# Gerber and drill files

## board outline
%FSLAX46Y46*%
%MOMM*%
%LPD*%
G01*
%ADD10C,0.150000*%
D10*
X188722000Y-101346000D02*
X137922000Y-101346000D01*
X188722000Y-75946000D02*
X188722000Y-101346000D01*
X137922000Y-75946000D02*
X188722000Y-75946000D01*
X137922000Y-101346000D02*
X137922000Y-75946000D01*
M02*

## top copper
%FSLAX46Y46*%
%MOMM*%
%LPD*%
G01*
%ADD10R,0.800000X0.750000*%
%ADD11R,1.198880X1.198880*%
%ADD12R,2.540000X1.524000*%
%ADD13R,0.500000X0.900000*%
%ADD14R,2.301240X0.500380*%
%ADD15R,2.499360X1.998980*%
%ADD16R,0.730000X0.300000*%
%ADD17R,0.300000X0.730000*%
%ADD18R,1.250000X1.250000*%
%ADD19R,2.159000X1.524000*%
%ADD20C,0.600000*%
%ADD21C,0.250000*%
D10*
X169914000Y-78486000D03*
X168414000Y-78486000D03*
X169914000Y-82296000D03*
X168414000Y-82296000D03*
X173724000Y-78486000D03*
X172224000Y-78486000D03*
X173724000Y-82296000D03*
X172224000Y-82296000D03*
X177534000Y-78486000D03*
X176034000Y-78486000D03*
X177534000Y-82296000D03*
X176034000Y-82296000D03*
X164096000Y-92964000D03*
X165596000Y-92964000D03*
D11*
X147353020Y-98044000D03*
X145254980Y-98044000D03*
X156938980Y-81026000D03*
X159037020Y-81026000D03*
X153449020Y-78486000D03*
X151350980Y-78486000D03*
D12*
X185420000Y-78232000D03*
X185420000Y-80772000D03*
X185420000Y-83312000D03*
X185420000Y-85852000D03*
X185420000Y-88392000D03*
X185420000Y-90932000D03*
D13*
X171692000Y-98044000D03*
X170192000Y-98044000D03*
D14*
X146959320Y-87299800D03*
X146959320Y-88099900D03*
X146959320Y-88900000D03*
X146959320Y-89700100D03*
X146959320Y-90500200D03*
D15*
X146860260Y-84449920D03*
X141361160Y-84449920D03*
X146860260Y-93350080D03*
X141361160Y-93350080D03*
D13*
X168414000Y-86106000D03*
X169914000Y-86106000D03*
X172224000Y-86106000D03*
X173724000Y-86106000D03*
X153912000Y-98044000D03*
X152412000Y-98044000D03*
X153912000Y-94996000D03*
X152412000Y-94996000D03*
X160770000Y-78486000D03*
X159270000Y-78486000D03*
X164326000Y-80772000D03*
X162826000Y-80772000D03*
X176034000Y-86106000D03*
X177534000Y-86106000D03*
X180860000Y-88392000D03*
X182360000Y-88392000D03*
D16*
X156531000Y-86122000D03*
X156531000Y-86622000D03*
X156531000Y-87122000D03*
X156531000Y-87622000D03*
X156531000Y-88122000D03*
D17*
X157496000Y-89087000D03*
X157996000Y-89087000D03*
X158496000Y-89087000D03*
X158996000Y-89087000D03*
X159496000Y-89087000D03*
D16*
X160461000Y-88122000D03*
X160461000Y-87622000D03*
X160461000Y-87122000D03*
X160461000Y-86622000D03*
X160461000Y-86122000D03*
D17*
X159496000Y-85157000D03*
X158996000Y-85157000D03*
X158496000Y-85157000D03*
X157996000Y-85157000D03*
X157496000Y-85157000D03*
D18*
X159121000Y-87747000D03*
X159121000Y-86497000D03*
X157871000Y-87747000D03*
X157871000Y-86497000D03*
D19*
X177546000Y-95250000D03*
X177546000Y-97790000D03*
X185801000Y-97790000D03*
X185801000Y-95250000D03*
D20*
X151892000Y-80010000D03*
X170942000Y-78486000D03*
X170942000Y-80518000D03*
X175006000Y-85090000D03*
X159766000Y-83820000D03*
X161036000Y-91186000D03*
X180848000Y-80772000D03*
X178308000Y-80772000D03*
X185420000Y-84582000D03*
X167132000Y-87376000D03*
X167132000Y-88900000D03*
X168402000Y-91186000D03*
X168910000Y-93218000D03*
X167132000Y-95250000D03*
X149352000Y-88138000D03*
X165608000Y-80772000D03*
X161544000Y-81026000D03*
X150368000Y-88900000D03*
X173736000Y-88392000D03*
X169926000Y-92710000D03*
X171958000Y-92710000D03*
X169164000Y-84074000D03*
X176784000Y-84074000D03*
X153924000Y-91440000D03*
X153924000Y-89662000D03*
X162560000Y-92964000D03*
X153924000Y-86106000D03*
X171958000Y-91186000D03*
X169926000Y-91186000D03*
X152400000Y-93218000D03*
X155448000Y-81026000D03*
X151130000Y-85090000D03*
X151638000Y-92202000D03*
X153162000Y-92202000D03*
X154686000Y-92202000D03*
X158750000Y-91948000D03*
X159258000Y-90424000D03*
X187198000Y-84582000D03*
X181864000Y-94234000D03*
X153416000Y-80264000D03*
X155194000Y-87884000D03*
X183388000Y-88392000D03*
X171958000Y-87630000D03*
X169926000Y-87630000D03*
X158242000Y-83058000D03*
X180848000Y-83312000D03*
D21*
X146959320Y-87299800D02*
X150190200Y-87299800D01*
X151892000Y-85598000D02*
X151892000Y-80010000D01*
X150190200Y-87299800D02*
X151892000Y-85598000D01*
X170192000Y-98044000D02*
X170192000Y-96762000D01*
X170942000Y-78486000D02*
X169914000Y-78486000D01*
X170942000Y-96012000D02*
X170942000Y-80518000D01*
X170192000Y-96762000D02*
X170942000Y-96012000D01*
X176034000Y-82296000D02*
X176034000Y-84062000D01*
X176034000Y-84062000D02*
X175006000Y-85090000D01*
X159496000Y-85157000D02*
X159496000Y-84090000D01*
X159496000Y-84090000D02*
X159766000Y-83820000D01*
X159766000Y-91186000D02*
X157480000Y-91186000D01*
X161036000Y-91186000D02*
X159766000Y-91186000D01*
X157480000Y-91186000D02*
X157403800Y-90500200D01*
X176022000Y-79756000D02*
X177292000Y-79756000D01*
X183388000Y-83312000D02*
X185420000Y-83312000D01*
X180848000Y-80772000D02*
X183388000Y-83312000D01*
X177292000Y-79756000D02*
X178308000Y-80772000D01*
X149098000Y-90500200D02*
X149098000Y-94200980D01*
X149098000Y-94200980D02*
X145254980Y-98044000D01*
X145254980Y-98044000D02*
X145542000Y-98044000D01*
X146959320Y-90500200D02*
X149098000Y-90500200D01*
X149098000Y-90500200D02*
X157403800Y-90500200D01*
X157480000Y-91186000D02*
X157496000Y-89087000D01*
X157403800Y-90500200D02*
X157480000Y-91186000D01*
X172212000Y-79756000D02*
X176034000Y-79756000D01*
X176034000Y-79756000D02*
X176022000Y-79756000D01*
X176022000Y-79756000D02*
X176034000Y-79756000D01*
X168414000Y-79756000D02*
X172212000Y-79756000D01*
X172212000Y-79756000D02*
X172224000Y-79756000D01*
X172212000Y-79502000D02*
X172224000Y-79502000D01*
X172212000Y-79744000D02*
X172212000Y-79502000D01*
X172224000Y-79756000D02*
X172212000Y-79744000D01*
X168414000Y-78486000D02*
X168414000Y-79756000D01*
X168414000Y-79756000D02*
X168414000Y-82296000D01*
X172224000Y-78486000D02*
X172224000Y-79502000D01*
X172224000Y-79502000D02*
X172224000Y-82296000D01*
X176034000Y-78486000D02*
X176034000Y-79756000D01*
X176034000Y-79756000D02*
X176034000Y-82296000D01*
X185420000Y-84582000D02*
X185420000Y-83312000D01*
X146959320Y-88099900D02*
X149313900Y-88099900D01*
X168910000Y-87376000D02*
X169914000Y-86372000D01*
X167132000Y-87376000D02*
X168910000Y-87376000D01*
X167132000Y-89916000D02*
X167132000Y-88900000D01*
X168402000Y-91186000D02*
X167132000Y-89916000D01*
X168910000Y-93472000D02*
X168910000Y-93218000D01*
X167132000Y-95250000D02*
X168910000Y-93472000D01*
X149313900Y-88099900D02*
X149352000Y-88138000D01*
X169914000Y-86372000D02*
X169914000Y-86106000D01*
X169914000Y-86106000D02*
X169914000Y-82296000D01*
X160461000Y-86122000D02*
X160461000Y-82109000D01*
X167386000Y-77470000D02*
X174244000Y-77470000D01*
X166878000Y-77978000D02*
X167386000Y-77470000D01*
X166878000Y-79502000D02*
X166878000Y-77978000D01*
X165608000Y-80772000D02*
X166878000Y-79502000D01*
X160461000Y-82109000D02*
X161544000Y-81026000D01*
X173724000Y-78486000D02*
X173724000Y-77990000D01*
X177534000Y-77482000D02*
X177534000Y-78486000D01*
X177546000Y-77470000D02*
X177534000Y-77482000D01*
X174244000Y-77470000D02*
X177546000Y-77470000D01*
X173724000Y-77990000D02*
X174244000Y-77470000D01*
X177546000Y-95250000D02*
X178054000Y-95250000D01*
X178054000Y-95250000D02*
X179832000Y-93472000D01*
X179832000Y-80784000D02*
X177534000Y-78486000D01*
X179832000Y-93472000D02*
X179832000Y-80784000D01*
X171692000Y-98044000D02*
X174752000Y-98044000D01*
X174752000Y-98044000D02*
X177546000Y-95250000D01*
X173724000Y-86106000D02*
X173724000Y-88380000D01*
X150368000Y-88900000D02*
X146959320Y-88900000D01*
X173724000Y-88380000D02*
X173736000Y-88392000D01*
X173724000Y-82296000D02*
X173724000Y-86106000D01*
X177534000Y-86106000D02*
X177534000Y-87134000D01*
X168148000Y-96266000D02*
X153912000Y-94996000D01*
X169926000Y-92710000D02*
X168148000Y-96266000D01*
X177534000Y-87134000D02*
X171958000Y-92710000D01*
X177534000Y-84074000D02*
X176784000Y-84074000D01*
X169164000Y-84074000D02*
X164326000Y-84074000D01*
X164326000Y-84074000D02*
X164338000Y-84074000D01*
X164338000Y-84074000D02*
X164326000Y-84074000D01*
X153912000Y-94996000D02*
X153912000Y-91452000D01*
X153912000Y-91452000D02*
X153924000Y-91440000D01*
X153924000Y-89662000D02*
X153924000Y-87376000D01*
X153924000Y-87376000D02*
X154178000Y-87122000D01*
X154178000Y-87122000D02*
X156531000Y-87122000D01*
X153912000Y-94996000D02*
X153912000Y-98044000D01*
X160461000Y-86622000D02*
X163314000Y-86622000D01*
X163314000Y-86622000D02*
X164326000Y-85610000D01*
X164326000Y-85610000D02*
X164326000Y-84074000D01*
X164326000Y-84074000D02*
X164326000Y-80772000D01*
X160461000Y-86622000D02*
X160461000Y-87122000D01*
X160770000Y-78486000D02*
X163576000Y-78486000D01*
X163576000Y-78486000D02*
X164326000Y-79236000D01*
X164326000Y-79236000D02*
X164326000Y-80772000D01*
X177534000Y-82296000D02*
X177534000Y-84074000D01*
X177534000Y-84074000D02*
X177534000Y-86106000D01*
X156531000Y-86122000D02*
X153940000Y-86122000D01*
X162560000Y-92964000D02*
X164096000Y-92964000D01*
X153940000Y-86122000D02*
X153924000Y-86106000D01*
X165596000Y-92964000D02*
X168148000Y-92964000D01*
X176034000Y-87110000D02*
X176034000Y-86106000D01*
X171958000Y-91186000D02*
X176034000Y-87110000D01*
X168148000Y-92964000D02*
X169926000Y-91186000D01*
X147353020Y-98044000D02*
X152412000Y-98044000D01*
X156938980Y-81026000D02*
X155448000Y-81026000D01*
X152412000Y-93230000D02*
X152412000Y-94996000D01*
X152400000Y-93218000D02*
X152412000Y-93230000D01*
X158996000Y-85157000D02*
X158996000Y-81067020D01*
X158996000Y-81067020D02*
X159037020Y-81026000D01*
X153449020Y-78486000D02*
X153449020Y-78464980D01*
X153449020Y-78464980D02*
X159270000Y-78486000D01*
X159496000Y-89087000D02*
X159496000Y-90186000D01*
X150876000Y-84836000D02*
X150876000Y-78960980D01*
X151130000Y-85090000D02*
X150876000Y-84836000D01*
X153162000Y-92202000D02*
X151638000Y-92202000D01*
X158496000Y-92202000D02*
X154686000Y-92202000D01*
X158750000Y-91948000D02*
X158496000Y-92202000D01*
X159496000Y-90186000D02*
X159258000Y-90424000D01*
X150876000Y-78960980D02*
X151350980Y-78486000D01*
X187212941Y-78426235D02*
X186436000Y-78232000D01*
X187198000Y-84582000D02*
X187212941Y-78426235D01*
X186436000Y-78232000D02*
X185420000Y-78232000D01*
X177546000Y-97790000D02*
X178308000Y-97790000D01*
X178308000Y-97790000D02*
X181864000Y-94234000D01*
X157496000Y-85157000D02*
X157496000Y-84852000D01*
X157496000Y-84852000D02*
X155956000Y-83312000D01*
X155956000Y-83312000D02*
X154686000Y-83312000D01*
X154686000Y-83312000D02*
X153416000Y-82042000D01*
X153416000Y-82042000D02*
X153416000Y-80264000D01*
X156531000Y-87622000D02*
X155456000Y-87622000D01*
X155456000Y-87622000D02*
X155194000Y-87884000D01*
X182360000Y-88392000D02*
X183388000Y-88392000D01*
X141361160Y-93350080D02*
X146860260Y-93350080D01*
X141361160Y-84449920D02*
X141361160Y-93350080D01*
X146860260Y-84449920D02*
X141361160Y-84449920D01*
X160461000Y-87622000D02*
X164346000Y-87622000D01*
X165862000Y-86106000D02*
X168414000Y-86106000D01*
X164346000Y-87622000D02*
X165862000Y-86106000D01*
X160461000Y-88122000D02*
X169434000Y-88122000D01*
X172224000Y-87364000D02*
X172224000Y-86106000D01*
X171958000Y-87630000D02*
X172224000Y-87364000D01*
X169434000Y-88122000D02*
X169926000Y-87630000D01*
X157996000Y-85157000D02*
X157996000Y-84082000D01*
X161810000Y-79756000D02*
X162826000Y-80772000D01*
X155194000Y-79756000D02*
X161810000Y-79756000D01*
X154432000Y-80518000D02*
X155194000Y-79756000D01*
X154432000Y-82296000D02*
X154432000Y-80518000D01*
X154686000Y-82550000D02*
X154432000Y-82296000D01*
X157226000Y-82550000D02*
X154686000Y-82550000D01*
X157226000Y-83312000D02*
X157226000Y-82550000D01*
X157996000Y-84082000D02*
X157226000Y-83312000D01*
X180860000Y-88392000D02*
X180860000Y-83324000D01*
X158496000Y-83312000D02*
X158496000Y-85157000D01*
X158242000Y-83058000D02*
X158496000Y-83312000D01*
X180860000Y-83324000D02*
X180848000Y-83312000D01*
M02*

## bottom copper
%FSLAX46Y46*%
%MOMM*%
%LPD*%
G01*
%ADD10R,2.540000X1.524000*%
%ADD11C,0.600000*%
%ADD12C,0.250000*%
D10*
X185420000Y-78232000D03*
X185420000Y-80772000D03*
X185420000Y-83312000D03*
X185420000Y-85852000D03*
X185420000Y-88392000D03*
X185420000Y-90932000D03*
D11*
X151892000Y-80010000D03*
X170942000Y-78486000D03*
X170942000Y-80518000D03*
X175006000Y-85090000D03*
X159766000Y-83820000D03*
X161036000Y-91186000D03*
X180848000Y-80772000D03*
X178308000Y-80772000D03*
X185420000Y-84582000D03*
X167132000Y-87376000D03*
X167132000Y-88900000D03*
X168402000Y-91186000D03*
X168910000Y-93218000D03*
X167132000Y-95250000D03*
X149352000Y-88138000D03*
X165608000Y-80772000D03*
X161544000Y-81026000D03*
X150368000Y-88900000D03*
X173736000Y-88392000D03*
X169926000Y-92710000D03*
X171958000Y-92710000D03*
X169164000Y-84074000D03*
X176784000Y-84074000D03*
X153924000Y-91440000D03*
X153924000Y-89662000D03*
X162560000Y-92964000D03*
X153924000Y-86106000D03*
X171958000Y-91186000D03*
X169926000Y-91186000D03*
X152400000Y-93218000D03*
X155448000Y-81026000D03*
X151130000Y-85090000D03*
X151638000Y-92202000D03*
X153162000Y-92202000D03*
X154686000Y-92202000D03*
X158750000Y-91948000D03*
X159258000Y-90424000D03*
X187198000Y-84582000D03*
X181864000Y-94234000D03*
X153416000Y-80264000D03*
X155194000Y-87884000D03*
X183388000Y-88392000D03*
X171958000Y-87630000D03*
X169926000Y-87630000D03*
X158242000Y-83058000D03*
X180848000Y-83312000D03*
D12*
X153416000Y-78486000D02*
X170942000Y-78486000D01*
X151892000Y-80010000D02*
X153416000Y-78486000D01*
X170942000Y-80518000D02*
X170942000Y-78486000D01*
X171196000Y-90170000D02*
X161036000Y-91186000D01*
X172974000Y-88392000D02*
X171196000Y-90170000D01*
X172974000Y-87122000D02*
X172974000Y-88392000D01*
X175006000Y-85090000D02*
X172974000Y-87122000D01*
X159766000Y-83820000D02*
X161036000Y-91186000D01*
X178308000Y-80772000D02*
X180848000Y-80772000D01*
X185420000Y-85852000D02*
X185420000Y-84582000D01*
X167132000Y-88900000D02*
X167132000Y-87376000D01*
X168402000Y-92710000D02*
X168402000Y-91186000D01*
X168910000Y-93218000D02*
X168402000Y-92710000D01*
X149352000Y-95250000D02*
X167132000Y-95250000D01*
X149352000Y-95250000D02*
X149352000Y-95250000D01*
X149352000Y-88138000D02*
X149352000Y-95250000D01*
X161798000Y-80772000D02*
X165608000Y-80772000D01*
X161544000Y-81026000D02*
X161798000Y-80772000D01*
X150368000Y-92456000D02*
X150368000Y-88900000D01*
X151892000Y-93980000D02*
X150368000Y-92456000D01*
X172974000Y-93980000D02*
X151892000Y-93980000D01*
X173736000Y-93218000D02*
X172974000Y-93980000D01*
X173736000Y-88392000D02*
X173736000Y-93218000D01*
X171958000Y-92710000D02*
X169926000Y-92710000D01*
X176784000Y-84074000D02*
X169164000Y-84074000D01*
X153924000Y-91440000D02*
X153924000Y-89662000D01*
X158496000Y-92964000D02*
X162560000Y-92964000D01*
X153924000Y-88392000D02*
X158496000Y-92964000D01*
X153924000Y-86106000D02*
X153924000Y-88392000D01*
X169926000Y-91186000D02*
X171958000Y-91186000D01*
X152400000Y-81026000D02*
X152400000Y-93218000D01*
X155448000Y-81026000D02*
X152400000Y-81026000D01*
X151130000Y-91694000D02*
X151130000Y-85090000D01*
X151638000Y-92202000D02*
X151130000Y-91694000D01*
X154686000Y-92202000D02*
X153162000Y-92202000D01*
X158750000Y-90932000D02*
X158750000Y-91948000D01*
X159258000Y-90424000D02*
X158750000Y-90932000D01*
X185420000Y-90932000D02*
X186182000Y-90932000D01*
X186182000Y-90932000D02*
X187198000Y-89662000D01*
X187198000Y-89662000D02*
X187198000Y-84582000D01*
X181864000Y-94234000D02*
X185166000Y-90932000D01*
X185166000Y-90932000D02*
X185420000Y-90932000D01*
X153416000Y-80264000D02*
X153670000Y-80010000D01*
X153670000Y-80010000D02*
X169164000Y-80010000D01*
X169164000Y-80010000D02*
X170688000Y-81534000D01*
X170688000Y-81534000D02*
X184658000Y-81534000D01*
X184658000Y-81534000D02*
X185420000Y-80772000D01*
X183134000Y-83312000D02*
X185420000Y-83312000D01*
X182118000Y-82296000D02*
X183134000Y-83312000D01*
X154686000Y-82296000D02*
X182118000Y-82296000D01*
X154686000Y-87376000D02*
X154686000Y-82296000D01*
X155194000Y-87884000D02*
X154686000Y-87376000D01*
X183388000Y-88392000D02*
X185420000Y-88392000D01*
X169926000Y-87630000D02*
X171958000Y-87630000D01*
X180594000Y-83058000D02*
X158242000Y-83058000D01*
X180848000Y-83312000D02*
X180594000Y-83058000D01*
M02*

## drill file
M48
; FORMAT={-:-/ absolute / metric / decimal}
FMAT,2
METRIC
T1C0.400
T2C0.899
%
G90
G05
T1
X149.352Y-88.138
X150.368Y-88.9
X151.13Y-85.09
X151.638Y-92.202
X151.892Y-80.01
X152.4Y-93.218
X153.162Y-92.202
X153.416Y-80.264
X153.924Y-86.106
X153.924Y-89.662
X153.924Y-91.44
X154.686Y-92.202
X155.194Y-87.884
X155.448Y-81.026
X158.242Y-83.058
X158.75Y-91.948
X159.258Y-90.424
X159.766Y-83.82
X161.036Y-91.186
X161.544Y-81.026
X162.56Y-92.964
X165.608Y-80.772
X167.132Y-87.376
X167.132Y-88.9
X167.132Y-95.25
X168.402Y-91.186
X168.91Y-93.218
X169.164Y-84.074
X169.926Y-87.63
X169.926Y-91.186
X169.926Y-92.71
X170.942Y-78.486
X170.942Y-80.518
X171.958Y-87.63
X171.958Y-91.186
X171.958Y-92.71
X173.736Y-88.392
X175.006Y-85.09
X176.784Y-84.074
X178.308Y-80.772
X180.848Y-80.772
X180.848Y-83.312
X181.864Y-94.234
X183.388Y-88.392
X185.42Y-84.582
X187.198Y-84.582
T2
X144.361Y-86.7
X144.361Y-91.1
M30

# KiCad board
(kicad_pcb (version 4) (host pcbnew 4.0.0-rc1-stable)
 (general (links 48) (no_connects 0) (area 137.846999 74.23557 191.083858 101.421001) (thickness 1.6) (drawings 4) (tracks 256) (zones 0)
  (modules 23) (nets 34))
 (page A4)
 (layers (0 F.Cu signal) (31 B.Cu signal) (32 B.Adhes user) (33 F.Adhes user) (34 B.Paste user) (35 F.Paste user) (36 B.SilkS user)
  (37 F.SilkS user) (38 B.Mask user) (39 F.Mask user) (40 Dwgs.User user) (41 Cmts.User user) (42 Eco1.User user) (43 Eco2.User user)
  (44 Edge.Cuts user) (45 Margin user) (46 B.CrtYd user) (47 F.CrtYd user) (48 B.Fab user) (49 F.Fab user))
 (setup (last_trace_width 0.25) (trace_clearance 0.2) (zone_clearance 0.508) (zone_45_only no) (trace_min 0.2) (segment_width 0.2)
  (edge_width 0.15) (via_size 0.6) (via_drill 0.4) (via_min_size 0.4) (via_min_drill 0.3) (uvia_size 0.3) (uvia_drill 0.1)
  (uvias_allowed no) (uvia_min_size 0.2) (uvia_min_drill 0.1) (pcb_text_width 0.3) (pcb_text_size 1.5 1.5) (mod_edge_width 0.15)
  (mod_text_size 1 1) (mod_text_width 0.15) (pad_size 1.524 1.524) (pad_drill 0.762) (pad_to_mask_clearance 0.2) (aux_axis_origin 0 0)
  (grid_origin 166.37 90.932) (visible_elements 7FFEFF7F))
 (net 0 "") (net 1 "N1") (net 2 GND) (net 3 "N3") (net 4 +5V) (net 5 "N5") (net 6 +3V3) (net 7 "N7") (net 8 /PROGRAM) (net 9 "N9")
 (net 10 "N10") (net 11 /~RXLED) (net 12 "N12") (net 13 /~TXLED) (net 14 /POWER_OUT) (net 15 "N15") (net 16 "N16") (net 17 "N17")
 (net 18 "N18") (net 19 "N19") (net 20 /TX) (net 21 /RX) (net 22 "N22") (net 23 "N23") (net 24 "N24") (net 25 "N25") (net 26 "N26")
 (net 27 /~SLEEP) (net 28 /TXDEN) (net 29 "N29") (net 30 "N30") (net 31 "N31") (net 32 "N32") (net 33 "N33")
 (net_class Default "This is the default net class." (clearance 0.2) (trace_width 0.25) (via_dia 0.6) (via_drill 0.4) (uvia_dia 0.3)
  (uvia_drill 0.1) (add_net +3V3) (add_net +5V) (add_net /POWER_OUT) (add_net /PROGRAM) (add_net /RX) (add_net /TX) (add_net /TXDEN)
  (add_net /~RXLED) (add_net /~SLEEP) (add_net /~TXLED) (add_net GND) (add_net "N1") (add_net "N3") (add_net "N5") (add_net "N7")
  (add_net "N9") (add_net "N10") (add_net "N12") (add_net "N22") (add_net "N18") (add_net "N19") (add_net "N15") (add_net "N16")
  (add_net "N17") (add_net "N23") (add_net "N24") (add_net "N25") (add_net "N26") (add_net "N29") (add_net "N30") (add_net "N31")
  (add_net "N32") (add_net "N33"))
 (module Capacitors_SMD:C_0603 (layer F.Cu) (at 169.164 78.486 180)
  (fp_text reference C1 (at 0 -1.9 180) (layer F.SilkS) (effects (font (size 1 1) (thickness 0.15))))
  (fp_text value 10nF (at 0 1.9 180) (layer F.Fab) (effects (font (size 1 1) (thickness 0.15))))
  (pad 1 smd rect (at -0.75 0 180) (size 0.8 0.75) (layers F.Cu F.Paste F.Mask) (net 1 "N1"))
  (pad 2 smd rect (at 0.75 0 180) (size 0.8 0.75) (layers F.Cu F.Paste F.Mask) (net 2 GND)))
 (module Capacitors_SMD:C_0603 (layer F.Cu) (at 169.164 82.296 180)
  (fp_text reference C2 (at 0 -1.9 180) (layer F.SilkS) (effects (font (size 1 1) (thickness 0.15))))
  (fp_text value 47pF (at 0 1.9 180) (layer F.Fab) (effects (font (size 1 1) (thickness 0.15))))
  (pad 1 smd rect (at -0.75 0 180) (size 0.8 0.75) (layers F.Cu F.Paste F.Mask) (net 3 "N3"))
  (pad 2 smd rect (at 0.75 0 180) (size 0.8 0.75) (layers F.Cu F.Paste F.Mask) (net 2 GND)))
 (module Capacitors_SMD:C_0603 (layer F.Cu) (at 172.974 78.486 180)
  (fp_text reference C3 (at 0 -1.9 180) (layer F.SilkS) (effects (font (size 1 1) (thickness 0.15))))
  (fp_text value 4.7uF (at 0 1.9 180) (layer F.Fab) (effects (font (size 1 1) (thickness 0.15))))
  (pad 1 smd rect (at -0.75 0 180) (size 0.8 0.75) (layers F.Cu F.Paste F.Mask) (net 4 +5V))
  (pad 2 smd rect (at 0.75 0 180) (size 0.8 0.75) (layers F.Cu F.Paste F.Mask) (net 2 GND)))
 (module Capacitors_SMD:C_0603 (layer F.Cu) (at 172.974 82.296 180)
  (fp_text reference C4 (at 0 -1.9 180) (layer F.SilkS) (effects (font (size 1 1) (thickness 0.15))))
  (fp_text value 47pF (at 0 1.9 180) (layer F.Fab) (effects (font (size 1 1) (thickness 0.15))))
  (pad 1 smd rect (at -0.75 0 180) (size 0.8 0.75) (layers F.Cu F.Paste F.Mask) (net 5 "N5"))
  (pad 2 smd rect (at 0.75 0 180) (size 0.8 0.75) (layers F.Cu F.Paste F.Mask) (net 2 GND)))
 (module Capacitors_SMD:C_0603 (layer F.Cu) (at 176.784 78.486 180)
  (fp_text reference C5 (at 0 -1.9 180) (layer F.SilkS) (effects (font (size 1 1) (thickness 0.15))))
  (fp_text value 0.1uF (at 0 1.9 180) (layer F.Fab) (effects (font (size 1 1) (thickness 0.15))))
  (pad 1 smd rect (at -0.75 0 180) (size 0.8 0.75) (layers F.Cu F.Paste F.Mask) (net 4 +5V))
  (pad 2 smd rect (at 0.75 0 180) (size 0.8 0.75) (layers F.Cu F.Paste F.Mask) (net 2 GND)))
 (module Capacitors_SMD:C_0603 (layer F.Cu) (at 176.784 82.296 180)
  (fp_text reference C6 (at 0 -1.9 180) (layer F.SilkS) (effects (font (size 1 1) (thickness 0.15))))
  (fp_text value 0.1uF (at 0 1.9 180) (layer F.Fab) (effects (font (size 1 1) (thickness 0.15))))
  (pad 1 smd rect (at -0.75 0 180) (size 0.8 0.75) (layers F.Cu F.Paste F.Mask) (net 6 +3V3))
  (pad 2 smd rect (at 0.75 0 180) (size 0.8 0.75) (layers F.Cu F.Paste F.Mask) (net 2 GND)))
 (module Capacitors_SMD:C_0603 (layer F.Cu) (at 164.846 92.964)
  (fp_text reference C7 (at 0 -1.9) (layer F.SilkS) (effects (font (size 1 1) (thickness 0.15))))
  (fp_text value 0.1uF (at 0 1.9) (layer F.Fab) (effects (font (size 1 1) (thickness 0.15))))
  (pad 1 smd rect (at -0.75 0) (size 0.8 0.75) (layers F.Cu F.Paste F.Mask) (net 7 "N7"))
  (pad 2 smd rect (at 0.75 0) (size 0.8 0.75) (layers F.Cu F.Paste F.Mask) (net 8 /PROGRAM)))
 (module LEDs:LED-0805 (layer F.Cu) (at 146.304 98.044)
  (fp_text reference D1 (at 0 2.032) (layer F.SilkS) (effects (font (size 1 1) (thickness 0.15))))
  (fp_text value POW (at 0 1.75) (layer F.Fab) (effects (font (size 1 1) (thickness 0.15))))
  (pad 2 smd rect (at 1.04902 0 180) (size 1.19888 1.19888) (layers F.Cu F.Paste F.Mask) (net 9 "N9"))
  (pad 1 smd rect (at -1.04902 0 180) (size 1.19888 1.19888) (layers F.Cu F.Paste F.Mask) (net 2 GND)))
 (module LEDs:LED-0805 (layer F.Cu) (at 157.988 81.026 180)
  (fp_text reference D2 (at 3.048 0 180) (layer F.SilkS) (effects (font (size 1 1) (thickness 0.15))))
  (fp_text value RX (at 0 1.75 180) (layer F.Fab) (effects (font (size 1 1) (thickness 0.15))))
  (pad 2 smd rect (at 1.04902 0) (size 1.19888 1.19888) (layers F.Cu F.Paste F.Mask) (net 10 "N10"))
  (pad 1 smd rect (at -1.04902 0) (size 1.19888 1.19888) (layers F.Cu F.Paste F.Mask) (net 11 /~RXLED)))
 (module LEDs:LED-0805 (layer F.Cu) (at 152.4 78.486)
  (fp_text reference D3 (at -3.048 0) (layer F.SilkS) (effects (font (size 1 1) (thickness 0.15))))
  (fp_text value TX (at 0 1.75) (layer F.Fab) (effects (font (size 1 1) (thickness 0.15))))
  (pad 2 smd rect (at 1.04902 0 180) (size 1.19888 1.19888) (layers F.Cu F.Paste F.Mask) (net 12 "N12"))
  (pad 1 smd rect (at -1.04902 0 180) (size 1.19888 1.19888) (layers F.Cu F.Paste F.Mask) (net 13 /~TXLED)))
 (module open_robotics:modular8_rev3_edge (layer F.Cu) (at 185.42 83.312 270)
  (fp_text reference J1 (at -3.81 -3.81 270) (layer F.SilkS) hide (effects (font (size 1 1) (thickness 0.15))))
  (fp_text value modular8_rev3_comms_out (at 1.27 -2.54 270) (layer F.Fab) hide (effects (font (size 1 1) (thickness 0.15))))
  (pad 1 smd rect (at -5.08 0 270) (size 1.524 2.54) (layers F.Cu F.Paste F.Mask) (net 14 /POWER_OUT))
  (pad 3 smd rect (at -2.54 0 270) (size 1.524 2.54) (layers F.Cu F.Paste F.Mask) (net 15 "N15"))
  (pad 5 smd rect (at 0 0 270) (size 1.524 2.54) (layers F.Cu F.Paste F.Mask) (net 2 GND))
  (pad 7 smd rect (at 2.54 0 270) (size 1.524 2.54) (layers F.Cu F.Paste F.Mask) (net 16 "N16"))
  (pad 9 smd rect (at 5.08 0 270) (size 1.524 2.54) (layers F.Cu F.Paste F.Mask) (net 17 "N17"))
  (pad 11 smd rect (at 7.62 0 270) (size 1.524 2.54) (layers F.Cu F.Paste F.Mask) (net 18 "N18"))
  (pad 2 smd rect (at -5.08 0 270) (size 1.524 2.54) (layers B.Cu F.Paste F.Mask) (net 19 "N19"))
  (pad 4 smd rect (at -2.54 0 270) (size 1.524 2.54) (layers B.Cu F.Paste F.Mask) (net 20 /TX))
  (pad 6 smd rect (at 0 0 270) (size 1.524 2.54) (layers B.Cu F.Paste F.Mask) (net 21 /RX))
  (pad 8 smd rect (at 2.54 0 270) (size 1.524 2.54) (layers B.Cu F.Paste F.Mask) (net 2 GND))
  (pad 10 smd rect (at 5.08 0 270) (size 1.524 2.54) (layers B.Cu F.Paste F.Mask) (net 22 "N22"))
  (pad 12 smd rect (at 7.62 0 270) (size 1.524 2.54) (layers B.Cu F.Paste F.Mask) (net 14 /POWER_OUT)))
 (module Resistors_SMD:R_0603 (layer F.Cu) (at 170.942 98.044 180)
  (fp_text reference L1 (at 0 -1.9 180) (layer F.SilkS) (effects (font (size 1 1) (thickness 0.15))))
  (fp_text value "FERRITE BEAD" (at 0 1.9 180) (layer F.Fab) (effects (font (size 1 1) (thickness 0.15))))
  (pad 1 smd rect (at -0.75 0 180) (size 0.5 0.9) (layers F.Cu F.Paste F.Mask) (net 4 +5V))
  (pad 2 smd rect (at 0.75 0 180) (size 0.5 0.9) (layers F.Cu F.Paste F.Mask) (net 1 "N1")))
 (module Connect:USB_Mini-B (layer F.Cu) (at 143.51 88.9)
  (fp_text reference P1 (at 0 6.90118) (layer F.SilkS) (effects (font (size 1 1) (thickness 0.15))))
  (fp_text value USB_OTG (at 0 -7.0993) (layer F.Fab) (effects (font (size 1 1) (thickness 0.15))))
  (pad 1 smd rect (at 3.44932 -1.6002) (size 2.30124 0.50038) (layers F.Cu F.Paste F.Mask) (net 1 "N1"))
  (pad 2 smd rect (at 3.44932 -0.8001) (size 2.30124 0.50038) (layers F.Cu F.Paste F.Mask) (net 3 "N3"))
  (pad 3 smd rect (at 3.44932 0) (size 2.30124 0.50038) (layers F.Cu F.Paste F.Mask) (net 5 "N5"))
  (pad 4 smd rect (at 3.44932 0.8001) (size 2.30124 0.50038) (layers F.Cu F.Paste F.Mask) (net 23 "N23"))
  (pad 5 smd rect (at 3.44932 1.6002) (size 2.30124 0.50038) (layers F.Cu F.Paste F.Mask) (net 2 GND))
  (pad 6 smd rect (at 3.35026 -4.45008) (size 2.49936 1.99898) (layers F.Cu F.Paste F.Mask) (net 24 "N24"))
  (pad 6 smd rect (at -2.14884 -4.45008) (size 2.49936 1.99898) (layers F.Cu F.Paste F.Mask) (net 24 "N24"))
  (pad 6 smd rect (at 3.35026 4.45008) (size 2.49936 1.99898) (layers F.Cu F.Paste F.Mask) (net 24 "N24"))
  (pad 6 smd rect (at -2.14884 4.45008) (size 2.49936 1.99898) (layers F.Cu F.Paste F.Mask) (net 24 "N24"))
  (pad "" np_thru_hole circle (at 0.8509 -2.19964) (size 0.89916 0.89916) (drill 0.89916) (layers *.Cu *.Mask F.SilkS))
  (pad "" np_thru_hole circle (at 0.8509 2.19964) (size 0.89916 0.89916) (drill 0.89916) (layers *.Cu *.Mask F.SilkS)))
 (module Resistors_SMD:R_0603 (layer F.Cu) (at 169.164 86.106)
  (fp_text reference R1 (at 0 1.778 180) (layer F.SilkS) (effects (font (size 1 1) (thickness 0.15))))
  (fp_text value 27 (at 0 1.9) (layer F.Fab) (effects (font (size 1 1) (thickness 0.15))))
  (pad 1 smd rect (at -0.75 0) (size 0.5 0.9) (layers F.Cu F.Paste F.Mask) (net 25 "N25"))
  (pad 2 smd rect (at 0.75 0) (size 0.5 0.9) (layers F.Cu F.Paste F.Mask) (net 3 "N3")))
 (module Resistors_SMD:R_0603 (layer F.Cu) (at 172.974 86.106)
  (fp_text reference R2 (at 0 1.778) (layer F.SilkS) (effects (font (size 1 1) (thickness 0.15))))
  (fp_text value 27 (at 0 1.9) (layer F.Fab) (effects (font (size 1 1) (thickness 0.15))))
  (pad 1 smd rect (at -0.75 0) (size 0.5 0.9) (layers F.Cu F.Paste F.Mask) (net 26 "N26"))
  (pad 2 smd rect (at 0.75 0) (size 0.5 0.9) (layers F.Cu F.Paste F.Mask) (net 5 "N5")))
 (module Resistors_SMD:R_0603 (layer F.Cu) (at 153.162 98.044 180)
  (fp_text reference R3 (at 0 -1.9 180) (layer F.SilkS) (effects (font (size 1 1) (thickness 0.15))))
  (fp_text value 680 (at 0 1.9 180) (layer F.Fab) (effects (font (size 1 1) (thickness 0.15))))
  (pad 1 smd rect (at -0.75 0 180) (size 0.5 0.9) (layers F.Cu F.Paste F.Mask) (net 6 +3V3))
  (pad 2 smd rect (at 0.75 0 180) (size 0.5 0.9) (layers F.Cu F.Paste F.Mask) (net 9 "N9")))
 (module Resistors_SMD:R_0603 (layer F.Cu) (at 153.162 94.996 180)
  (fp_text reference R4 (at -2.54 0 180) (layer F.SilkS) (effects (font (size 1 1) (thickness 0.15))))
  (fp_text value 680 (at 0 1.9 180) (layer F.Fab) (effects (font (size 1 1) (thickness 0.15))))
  (pad 1 smd rect (at -0.75 0 180) (size 0.5 0.9) (layers F.Cu F.Paste F.Mask) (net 6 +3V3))
  (pad 2 smd rect (at 0.75 0 180) (size 0.5 0.9) (layers F.Cu F.Paste F.Mask) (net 10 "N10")))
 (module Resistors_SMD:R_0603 (layer F.Cu) (at 160.02 78.486 180)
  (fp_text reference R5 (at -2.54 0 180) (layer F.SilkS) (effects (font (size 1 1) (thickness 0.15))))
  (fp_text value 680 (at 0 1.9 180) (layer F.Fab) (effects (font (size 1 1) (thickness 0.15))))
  (pad 1 smd rect (at -0.75 0 180) (size 0.5 0.9) (layers F.Cu F.Paste F.Mask) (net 6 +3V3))
  (pad 2 smd rect (at 0.75 0 180) (size 0.5 0.9) (layers F.Cu F.Paste F.Mask) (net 12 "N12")))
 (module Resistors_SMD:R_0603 (layer F.Cu) (at 163.576 80.772 180)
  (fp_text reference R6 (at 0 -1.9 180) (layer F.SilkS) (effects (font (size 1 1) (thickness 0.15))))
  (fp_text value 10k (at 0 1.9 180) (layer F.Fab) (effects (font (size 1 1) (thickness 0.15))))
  (pad 1 smd rect (at -0.75 0 180) (size 0.5 0.9) (layers F.Cu F.Paste F.Mask) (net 6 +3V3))
  (pad 2 smd rect (at 0.75 0 180) (size 0.5 0.9) (layers F.Cu F.Paste F.Mask) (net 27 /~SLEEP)))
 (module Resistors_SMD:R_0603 (layer F.Cu) (at 176.784 86.106)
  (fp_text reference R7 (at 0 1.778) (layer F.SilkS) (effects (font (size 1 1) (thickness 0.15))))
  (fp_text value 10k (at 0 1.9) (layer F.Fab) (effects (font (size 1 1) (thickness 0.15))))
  (pad 1 smd rect (at -0.75 0) (size 0.5 0.9) (layers F.Cu F.Paste F.Mask) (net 8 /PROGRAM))
  (pad 2 smd rect (at 0.75 0) (size 0.5 0.9) (layers F.Cu F.Paste F.Mask) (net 6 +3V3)))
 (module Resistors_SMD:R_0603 (layer F.Cu) (at 181.61 88.392)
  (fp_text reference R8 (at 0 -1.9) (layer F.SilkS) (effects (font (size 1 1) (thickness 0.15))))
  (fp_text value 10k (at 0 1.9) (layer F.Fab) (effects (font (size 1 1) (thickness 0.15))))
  (pad 1 smd rect (at -0.75 0) (size 0.5 0.9) (layers F.Cu F.Paste F.Mask) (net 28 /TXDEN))
  (pad 2 smd rect (at 0.75 0) (size 0.5 0.9) (layers F.Cu F.Paste F.Mask) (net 22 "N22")))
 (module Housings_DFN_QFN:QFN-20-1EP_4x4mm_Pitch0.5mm (layer F.Cu) (at 158.496 87.122)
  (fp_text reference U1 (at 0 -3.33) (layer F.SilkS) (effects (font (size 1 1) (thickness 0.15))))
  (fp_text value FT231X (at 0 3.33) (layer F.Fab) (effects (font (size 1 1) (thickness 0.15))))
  (pad 1 smd rect (at -1.965 -1) (size 0.73 0.3) (layers F.Cu F.Paste F.Mask) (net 7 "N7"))
  (pad 2 smd rect (at -1.965 -0.5) (size 0.73 0.3) (layers F.Cu F.Paste F.Mask) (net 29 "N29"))
  (pad 3 smd rect (at -1.965 0) (size 0.73 0.3) (layers F.Cu F.Paste F.Mask) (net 6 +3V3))
  (pad 4 smd rect (at -1.965 0.5) (size 0.73 0.3) (layers F.Cu F.Paste F.Mask) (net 21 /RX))
  (pad 5 smd rect (at -1.965 1) (size 0.73 0.3) (layers F.Cu F.Paste F.Mask) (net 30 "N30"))
  (pad 6 smd rect (at -1 1.965 90) (size 0.73 0.3) (layers F.Cu F.Paste F.Mask) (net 2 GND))
  (pad 7 smd rect (at -0.5 1.965 90) (size 0.73 0.3) (layers F.Cu F.Paste F.Mask) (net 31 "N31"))
  (pad 8 smd rect (at 0 1.965 90) (size 0.73 0.3) (layers F.Cu F.Paste F.Mask) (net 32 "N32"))
  (pad 9 smd rect (at 0.5 1.965 90) (size 0.73 0.3) (layers F.Cu F.Paste F.Mask) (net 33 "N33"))
  (pad 10 smd rect (at 1 1.965 90) (size 0.73 0.3) (layers F.Cu F.Paste F.Mask) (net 13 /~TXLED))
  (pad 11 smd rect (at 1.965 1) (size 0.73 0.3) (layers F.Cu F.Paste F.Mask) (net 26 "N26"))
  (pad 12 smd rect (at 1.965 0.5) (size 0.73 0.3) (layers F.Cu F.Paste F.Mask) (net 25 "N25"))
  (pad 13 smd rect (at 1.965 0) (size 0.73 0.3) (layers F.Cu F.Paste F.Mask) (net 6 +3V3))
  (pad 14 smd rect (at 1.965 -0.5) (size 0.73 0.3) (layers F.Cu F.Paste F.Mask) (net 6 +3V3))
  (pad 15 smd rect (at 1.965 -1) (size 0.73 0.3) (layers F.Cu F.Paste F.Mask) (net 4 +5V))
  (pad 16 smd rect (at 1 -1.965 90) (size 0.73 0.3) (layers F.Cu F.Paste F.Mask) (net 2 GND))
  (pad 17 smd rect (at 0.5 -1.965 90) (size 0.73 0.3) (layers F.Cu F.Paste F.Mask) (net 11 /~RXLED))
  (pad 18 smd rect (at 0 -1.965 90) (size 0.73 0.3) (layers F.Cu F.Paste F.Mask) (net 28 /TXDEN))
  (pad 19 smd rect (at -0.5 -1.965 90) (size 0.73 0.3) (layers F.Cu F.Paste F.Mask) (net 27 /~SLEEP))
  (pad 20 smd rect (at -1 -1.965 90) (size 0.73 0.3) (layers F.Cu F.Paste F.Mask) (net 20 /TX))
  (pad 21 smd rect (at 0.625 0.625) (size 1.25 1.25) (layers F.Cu F.Paste F.Mask) (solder_paste_margin_ratio -0.2))
  (pad 21 smd rect (at 0.625 -0.625) (size 1.25 1.25) (layers F.Cu F.Paste F.Mask) (solder_paste_margin_ratio -0.2))
  (pad 21 smd rect (at -0.625 0.625) (size 1.25 1.25) (layers F.Cu F.Paste F.Mask) (solder_paste_margin_ratio -0.2))
  (pad 21 smd rect (at -0.625 -0.625) (size 1.25 1.25) (layers F.Cu F.Paste F.Mask) (solder_paste_margin_ratio -0.2)))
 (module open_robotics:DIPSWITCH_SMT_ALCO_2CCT (layer F.Cu) (at 177.546 95.25)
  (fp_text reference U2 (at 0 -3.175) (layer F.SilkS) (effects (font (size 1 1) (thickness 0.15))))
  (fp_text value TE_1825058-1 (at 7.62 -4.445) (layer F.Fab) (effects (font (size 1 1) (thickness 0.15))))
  (pad 1 smd rect (at 0 0) (size 2.159 1.524) (layers F.Cu F.Paste F.Mask) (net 4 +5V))
  (pad 2 smd rect (at 0 2.54) (size 2.159 1.524) (layers F.Cu F.Paste F.Mask) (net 14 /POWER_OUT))
  (pad 3 smd rect (at 8.255 2.54) (size 2.159 1.524) (layers F.Cu F.Paste F.Mask))
  (pad 4 smd rect (at 8.255 0) (size 2.159 1.524) (layers F.Cu F.Paste F.Mask)))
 (gr_line (start 188.722 101.346) (end 137.922 101.346) (angle 90) (layer Edge.Cuts) (width 0.15))
 (gr_line (start 188.722 75.946) (end 188.722 101.346) (angle 90) (layer Edge.Cuts) (width 0.15))
 (gr_line (start 137.922 75.946) (end 188.722 75.946) (angle 90) (layer Edge.Cuts) (width 0.15))
 (gr_line (start 137.922 101.346) (end 137.922 75.946) (angle 90) (layer Edge.Cuts) (width 0.15))
 (segment (start 146.95932 87.2998) (end 150.1902 87.2998) (width 0.25) (layer F.Cu) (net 1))
 (segment (start 153.416 78.486) (end 170.942 78.486) (width 0.25) (layer B.Cu) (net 1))
 (segment (start 151.892 80.01) (end 153.416 78.486) (width 0.25) (layer B.Cu) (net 1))
 (via (at 151.892 80.01) (size 0.6) (drill 0.4) (layers F.Cu B.Cu) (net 1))
 (segment (start 151.892 85.598) (end 151.892 80.01) (width 0.25) (layer F.Cu) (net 1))
 (segment (start 150.1902 87.2998) (end 151.892 85.598) (width 0.25) (layer F.Cu) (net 1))
 (segment (start 170.192 98.044) (end 170.192 96.762) (width 0.25) (layer F.Cu) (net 1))
 (segment (start 170.942 78.486) (end 169.914 78.486) (width 0.25) (layer F.Cu) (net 1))
 (via (at 170.942 78.486) (size 0.6) (drill 0.4) (layers F.Cu B.Cu) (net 1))
 (segment (start 170.942 80.518) (end 170.942 78.486) (width 0.25) (layer B.Cu) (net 1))
 (via (at 170.942 80.518) (size 0.6) (drill 0.4) (layers F.Cu B.Cu) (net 1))
 (segment (start 170.942 96.012) (end 170.942 80.518) (width 0.25) (layer F.Cu) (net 1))
 (segment (start 170.192 96.762) (end 170.942 96.012) (width 0.25) (layer F.Cu) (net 1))
 (segment (start 176.034 82.296) (end 176.034 84.062) (width 0.25) (layer F.Cu) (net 2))
 (segment (start 171.196 90.17) (end 161.036 91.186) (width 0.25) (layer B.Cu) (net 2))
 (segment (start 172.974 88.392) (end 171.196 90.17) (width 0.25) (layer B.Cu) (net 2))
 (segment (start 172.974 87.122) (end 172.974 88.392) (width 0.25) (layer B.Cu) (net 2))
 (segment (start 175.006 85.09) (end 172.974 87.122) (width 0.25) (layer B.Cu) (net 2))
 (via (at 175.006 85.09) (size 0.6) (drill 0.4) (layers F.Cu B.Cu) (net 2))
 (segment (start 176.034 84.062) (end 175.006 85.09) (width 0.25) (layer F.Cu) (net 2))
 (segment (start 159.496 85.157) (end 159.496 84.09) (width 0.25) (layer F.Cu) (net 2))
 (segment (start 159.496 84.09) (end 159.766 83.82) (width 0.25) (layer F.Cu) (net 2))
 (via (at 159.766 83.82) (size 0.6) (drill 0.4) (layers F.Cu B.Cu) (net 2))
 (segment (start 159.766 83.82) (end 161.036 91.186) (width 0.25) (layer B.Cu) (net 2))
 (segment (start 159.766 91.186) (end 157.48 91.186) (width 0.25) (layer F.Cu) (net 2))
 (via (at 161.036 91.186) (size 0.6) (drill 0.4) (layers F.Cu B.Cu) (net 2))
 (segment (start 161.036 91.186) (end 159.766 91.186) (width 0.25) (layer F.Cu) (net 2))
 (segment (start 157.48 91.186) (end 157.4038 90.5002) (width 0.25) (layer F.Cu) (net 2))
 (segment (start 176.022 79.756) (end 177.292 79.756) (width 0.25) (layer F.Cu) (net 2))
 (segment (start 183.388 83.312) (end 185.42 83.312) (width 0.25) (layer F.Cu) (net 2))
 (segment (start 180.848 80.772) (end 183.388 83.312) (width 0.25) (layer F.Cu) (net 2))
 (via (at 180.848 80.772) (size 0.6) (drill 0.4) (layers F.Cu B.Cu) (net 2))
 (segment (start 178.308 80.772) (end 180.848 80.772) (width 0.25) (layer B.Cu) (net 2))
 (via (at 178.308 80.772) (size 0.6) (drill 0.4) (layers F.Cu B.Cu) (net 2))
 (segment (start 177.292 79.756) (end 178.308 80.772) (width 0.25) (layer F.Cu) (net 2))
 (segment (start 149.098 90.5002) (end 149.098 94.20098) (width 0.25) (layer F.Cu) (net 2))
 (segment (start 149.098 94.20098) (end 145.25498 98.044) (width 0.25) (layer F.Cu) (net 2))
 (segment (start 145.25498 98.044) (end 145.542 98.044) (width 0.25) (layer F.Cu) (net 2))
 (segment (start 146.95932 90.5002) (end 149.098 90.5002) (width 0.25) (layer F.Cu) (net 2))
 (segment (start 149.098 90.5002) (end 157.4038 90.5002) (width 0.25) (layer F.Cu) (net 2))
 (segment (start 157.48 91.186) (end 157.496 89.087) (width 0.25) (layer F.Cu) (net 2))
 (segment (start 157.4038 90.5002) (end 157.48 91.186) (width 0.25) (layer F.Cu) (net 2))
 (segment (start 172.212 79.756) (end 176.034 79.756) (width 0.25) (layer F.Cu) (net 2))
 (segment (start 176.034 79.756) (end 176.022 79.756) (width 0.25) (layer F.Cu) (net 2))
 (segment (start 176.022 79.756) (end 176.034 79.756) (width 0.25) (layer F.Cu) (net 2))
 (segment (start 168.414 79.756) (end 172.212 79.756) (width 0.25) (layer F.Cu) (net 2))
 (segment (start 172.212 79.756) (end 172.224 79.756) (width 0.25) (layer F.Cu) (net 2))
 (segment (start 172.212 79.502) (end 172.224 79.502) (width 0.25) (layer F.Cu) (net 2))
 (segment (start 172.212 79.744) (end 172.212 79.502) (width 0.25) (layer F.Cu) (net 2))
 (segment (start 172.224 79.756) (end 172.212 79.744) (width 0.25) (layer F.Cu) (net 2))
 (segment (start 168.414 78.486) (end 168.414 79.756) (width 0.25) (layer F.Cu) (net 2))
 (segment (start 168.414 79.756) (end 168.414 82.296) (width 0.25) (layer F.Cu) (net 2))
 (segment (start 172.224 78.486) (end 172.224 79.502) (width 0.25) (layer F.Cu) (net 2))
 (segment (start 172.224 79.502) (end 172.224 82.296) (width 0.25) (layer F.Cu) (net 2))
 (segment (start 176.034 78.486) (end 176.034 79.756) (width 0.25) (layer F.Cu) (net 2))
 (segment (start 176.034 79.756) (end 176.034 82.296) (width 0.25) (layer F.Cu) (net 2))
 (segment (start 185.42 85.852) (end 185.42 84.582) (width 0.25) (layer B.Cu) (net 2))
 (via (at 185.42 84.582) (size 0.6) (drill 0.4) (layers F.Cu B.Cu) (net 2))
 (segment (start 185.42 84.582) (end 185.42 83.312) (width 0.25) (layer F.Cu) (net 2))
 (segment (start 146.95932 88.0999) (end 149.3139 88.0999) (width 0.25) (layer F.Cu) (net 3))
 (segment (start 168.91 87.376) (end 169.914 86.372) (width 0.25) (layer F.Cu) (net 3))
 (segment (start 167.132 87.376) (end 168.91 87.376) (width 0.25) (layer F.Cu) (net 3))
 (via (at 167.132 87.376) (size 0.6) (drill 0.4) (layers F.Cu B.Cu) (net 3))
 (segment (start 167.132 88.9) (end 167.132 87.376) (width 0.25) (layer B.Cu) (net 3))
 (via (at 167.132 88.9) (size 0.6) (drill 0.4) (layers F.Cu B.Cu) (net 3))
 (segment (start 167.132 89.916) (end 167.132 88.9) (width 0.25) (layer F.Cu) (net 3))
 (segment (start 168.402 91.186) (end 167.132 89.916) (width 0.25) (layer F.Cu) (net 3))
 (via (at 168.402 91.186) (size 0.6) (drill 0.4) (layers F.Cu B.Cu) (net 3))
 (segment (start 168.402 92.71) (end 168.402 91.186) (width 0.25) (layer B.Cu) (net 3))
 (segment (start 168.91 93.218) (end 168.402 92.71) (width 0.25) (layer B.Cu) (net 3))
 (via (at 168.91 93.218) (size 0.6) (drill 0.4) (layers F.Cu B.Cu) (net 3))
 (segment (start 168.91 93.472) (end 168.91 93.218) (width 0.25) (layer F.Cu) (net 3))
 (segment (start 167.132 95.25) (end 168.91 93.472) (width 0.25) (layer F.Cu) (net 3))
 (via (at 167.132 95.25) (size 0.6) (drill 0.4) (layers F.Cu B.Cu) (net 3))
 (segment (start 149.352 95.25) (end 167.132 95.25) (width 0.25) (layer B.Cu) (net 3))
 (segment (start 149.352 95.25) (end 149.352 95.25) (width 0.25) (layer B.Cu) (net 3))
 (segment (start 149.352 88.138) (end 149.352 95.25) (width 0.25) (layer B.Cu) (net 3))
 (via (at 149.352 88.138) (size 0.6) (drill 0.4) (layers F.Cu B.Cu) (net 3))
 (segment (start 149.3139 88.0999) (end 149.352 88.138) (width 0.25) (layer F.Cu) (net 3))
 (segment (start 169.914 86.372) (end 169.914 86.106) (width 0.25) (layer F.Cu) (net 3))
 (segment (start 169.914 86.106) (end 169.914 82.296) (width 0.25) (layer F.Cu) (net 3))
 (segment (start 160.461 86.122) (end 160.461 82.109) (width 0.25) (layer F.Cu) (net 4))
 (segment (start 167.386 77.47) (end 174.244 77.47) (width 0.25) (layer F.Cu) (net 4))
 (segment (start 166.878 77.978) (end 167.386 77.47) (width 0.25) (layer F.Cu) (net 4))
 (segment (start 166.878 79.502) (end 166.878 77.978) (width 0.25) (layer F.Cu) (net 4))
 (segment (start 165.608 80.772) (end 166.878 79.502) (width 0.25) (layer F.Cu) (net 4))
 (via (at 165.608 80.772) (size 0.6) (drill 0.4) (layers F.Cu B.Cu) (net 4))
 (segment (start 161.798 80.772) (end 165.608 80.772) (width 0.25) (layer B.Cu) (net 4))
 (segment (start 161.544 81.026) (end 161.798 80.772) (width 0.25) (layer B.Cu) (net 4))
 (via (at 161.544 81.026) (size 0.6) (drill 0.4) (layers F.Cu B.Cu) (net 4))
 (segment (start 160.461 82.109) (end 161.544 81.026) (width 0.25) (layer F.Cu) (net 4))
 (segment (start 173.724 78.486) (end 173.724 77.99) (width 0.25) (layer F.Cu) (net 4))
 (segment (start 177.534 77.482) (end 177.534 78.486) (width 0.25) (layer F.Cu) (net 4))
 (segment (start 177.546 77.47) (end 177.534 77.482) (width 0.25) (layer F.Cu) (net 4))
 (segment (start 174.244 77.47) (end 177.546 77.47) (width 0.25) (layer F.Cu) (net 4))
 (segment (start 173.724 77.99) (end 174.244 77.47) (width 0.25) (layer F.Cu) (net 4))
 (segment (start 177.546 95.25) (end 178.054 95.25) (width 0.25) (layer F.Cu) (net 4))
 (segment (start 178.054 95.25) (end 179.832 93.472) (width 0.25) (layer F.Cu) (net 4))
 (segment (start 179.832 80.784) (end 177.534 78.486) (width 0.25) (layer F.Cu) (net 4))
 (segment (start 179.832 93.472) (end 179.832 80.784) (width 0.25) (layer F.Cu) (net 4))
 (segment (start 171.692 98.044) (end 174.752 98.044) (width 0.25) (layer F.Cu) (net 4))
 (segment (start 174.752 98.044) (end 177.546 95.25) (width 0.25) (layer F.Cu) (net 4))
 (segment (start 173.724 86.106) (end 173.724 88.38) (width 0.25) (layer F.Cu) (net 5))
 (segment (start 150.368 88.9) (end 146.95932 88.9) (width 0.25) (layer F.Cu) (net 5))
 (via (at 150.368 88.9) (size 0.6) (drill 0.4) (layers F.Cu B.Cu) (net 5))
 (segment (start 150.368 92.456) (end 150.368 88.9) (width 0.25) (layer B.Cu) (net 5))
 (segment (start 151.892 93.98) (end 150.368 92.456) (width 0.25) (layer B.Cu) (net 5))
 (segment (start 172.974 93.98) (end 151.892 93.98) (width 0.25) (layer B.Cu) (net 5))
 (segment (start 173.736 93.218) (end 172.974 93.98) (width 0.25) (layer B.Cu) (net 5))
 (segment (start 173.736 88.392) (end 173.736 93.218) (width 0.25) (layer B.Cu) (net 5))
 (via (at 173.736 88.392) (size 0.6) (drill 0.4) (layers F.Cu B.Cu) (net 5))
 (segment (start 173.724 88.38) (end 173.736 88.392) (width 0.25) (layer F.Cu) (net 5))
 (segment (start 173.724 82.296) (end 173.724 86.106) (width 0.25) (layer F.Cu) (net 5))
 (segment (start 177.534 86.106) (end 177.534 87.134) (width 0.25) (layer F.Cu) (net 6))
 (segment (start 168.148 96.266) (end 153.912 94.996) (width 0.25) (layer F.Cu) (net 6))
 (segment (start 169.926 92.71) (end 168.148 96.266) (width 0.25) (layer F.Cu) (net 6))
 (via (at 169.926 92.71) (size 0.6) (drill 0.4) (layers F.Cu B.Cu) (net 6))
 (segment (start 171.958 92.71) (end 169.926 92.71) (width 0.25) (layer B.Cu) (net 6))
 (via (at 171.958 92.71) (size 0.6) (drill 0.4) (layers F.Cu B.Cu) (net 6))
 (segment (start 177.534 87.134) (end 171.958 92.71) (width 0.25) (layer F.Cu) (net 6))
 (segment (start 177.534 84.074) (end 176.784 84.074) (width 0.25) (layer F.Cu) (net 6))
 (segment (start 169.164 84.074) (end 164.326 84.074) (width 0.25) (layer F.Cu) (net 6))
 (via (at 169.164 84.074) (size 0.6) (drill 0.4) (layers F.Cu B.Cu) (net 6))
 (segment (start 176.784 84.074) (end 169.164 84.074) (width 0.25) (layer B.Cu) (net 6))
 (via (at 176.784 84.074) (size 0.6) (drill 0.4) (layers F.Cu B.Cu) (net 6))
 (segment (start 164.326 84.074) (end 164.338 84.074) (width 0.25) (layer F.Cu) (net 6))
 (segment (start 164.338 84.074) (end 164.326 84.074) (width 0.25) (layer F.Cu) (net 6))
 (segment (start 153.912 94.996) (end 153.912 91.452) (width 0.25) (layer F.Cu) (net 6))
 (segment (start 153.912 91.452) (end 153.924 91.44) (width 0.25) (layer F.Cu) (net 6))
 (via (at 153.924 91.44) (size 0.6) (drill 0.4) (layers F.Cu B.Cu) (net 6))
 (segment (start 153.924 91.44) (end 153.924 89.662) (width 0.25) (layer B.Cu) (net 6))
 (via (at 153.924 89.662) (size 0.6) (drill 0.4) (layers F.Cu B.Cu) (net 6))
 (segment (start 153.924 89.662) (end 153.924 87.376) (width 0.25) (layer F.Cu) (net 6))
 (segment (start 153.924 87.376) (end 154.178 87.122) (width 0.25) (layer F.Cu) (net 6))
 (segment (start 154.178 87.122) (end 156.531 87.122) (width 0.25) (layer F.Cu) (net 6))
 (segment (start 153.912 94.996) (end 153.912 98.044) (width 0.25) (layer F.Cu) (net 6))
 (segment (start 160.461 86.622) (end 163.314 86.622) (width 0.25) (layer F.Cu) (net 6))
 (segment (start 163.314 86.622) (end 164.326 85.61) (width 0.25) (layer F.Cu) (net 6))
 (segment (start 164.326 85.61) (end 164.326 84.074) (width 0.25) (layer F.Cu) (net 6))
 (segment (start 164.326 84.074) (end 164.326 80.772) (width 0.25) (layer F.Cu) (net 6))
 (segment (start 160.461 86.622) (end 160.461 87.122) (width 0.25) (layer F.Cu) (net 6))
 (segment (start 160.77 78.486) (end 163.576 78.486) (width 0.25) (layer F.Cu) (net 6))
 (segment (start 163.576 78.486) (end 164.326 79.236) (width 0.25) (layer F.Cu) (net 6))
 (segment (start 164.326 79.236) (end 164.326 80.772) (width 0.25) (layer F.Cu) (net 6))
 (segment (start 177.534 82.296) (end 177.534 84.074) (width 0.25) (layer F.Cu) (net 6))
 (segment (start 177.534 84.074) (end 177.534 86.106) (width 0.25) (layer F.Cu) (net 6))
 (segment (start 156.531 86.122) (end 153.94 86.122) (width 0.25) (layer F.Cu) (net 7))
 (segment (start 162.56 92.964) (end 164.096 92.964) (width 0.25) (layer F.Cu) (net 7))
 (via (at 162.56 92.964) (size 0.6) (drill 0.4) (layers F.Cu B.Cu) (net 7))
 (segment (start 158.496 92.964) (end 162.56 92.964) (width 0.25) (layer B.Cu) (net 7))
 (segment (start 153.924 88.392) (end 158.496 92.964) (width 0.25) (layer B.Cu) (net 7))
 (segment (start 153.924 86.106) (end 153.924 88.392) (width 0.25) (layer B.Cu) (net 7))
 (via (at 153.924 86.106) (size 0.6) (drill 0.4) (layers F.Cu B.Cu) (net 7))
 (segment (start 153.94 86.122) (end 153.924 86.106) (width 0.25) (layer F.Cu) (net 7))
 (segment (start 165.596 92.964) (end 168.148 92.964) (width 0.25) (layer F.Cu) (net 8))
 (segment (start 176.034 87.11) (end 176.034 86.106) (width 0.25) (layer F.Cu) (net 8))
 (segment (start 171.958 91.186) (end 176.034 87.11) (width 0.25) (layer F.Cu) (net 8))
 (via (at 171.958 91.186) (size 0.6) (drill 0.4) (layers F.Cu B.Cu) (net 8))
 (segment (start 169.926 91.186) (end 171.958 91.186) (width 0.25) (layer B.Cu) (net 8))
 (via (at 169.926 91.186) (size 0.6) (drill 0.4) (layers F.Cu B.Cu) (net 8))
 (segment (start 168.148 92.964) (end 169.926 91.186) (width 0.25) (layer F.Cu) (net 8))
 (segment (start 147.35302 98.044) (end 152.412 98.044) (width 0.25) (layer F.Cu) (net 9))
 (segment (start 156.93898 81.026) (end 155.448 81.026) (width 0.25) (layer F.Cu) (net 10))
 (segment (start 152.412 93.23) (end 152.412 94.996) (width 0.25) (layer F.Cu) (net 10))
 (segment (start 152.4 93.218) (end 152.412 93.23) (width 0.25) (layer F.Cu) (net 10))
 (via (at 152.4 93.218) (size 0.6) (drill 0.4) (layers F.Cu B.Cu) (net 10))
 (segment (start 152.4 81.026) (end 152.4 93.218) (width 0.25) (layer B.Cu) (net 10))
 (segment (start 155.448 81.026) (end 152.4 81.026) (width 0.25) (layer B.Cu) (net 10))
 (via (at 155.448 81.026) (size 0.6) (drill 0.4) (layers F.Cu B.Cu) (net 10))
 (segment (start 158.996 85.157) (end 158.996 81.06702) (width 0.25) (layer F.Cu) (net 11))
 (segment (start 158.996 81.06702) (end 159.03702 81.026) (width 0.25) (layer F.Cu) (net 11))
 (segment (start 153.44902 78.486) (end 153.44902 78.46498) (width 0.25) (layer F.Cu) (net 12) (status 30))
 (segment (start 153.44902 78.46498) (end 159.27 78.486) (width 0.25) (layer F.Cu) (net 12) (status 10))
 (segment (start 159.496 89.087) (end 159.496 90.186) (width 0.25) (layer F.Cu) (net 13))
 (segment (start 150.876 84.836) (end 150.876 78.96098) (width 0.25) (layer F.Cu) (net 13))
 (segment (start 151.13 85.09) (end 150.876 84.836) (width 0.25) (layer F.Cu) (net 13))
 (via (at 151.13 85.09) (size 0.6) (drill 0.4) (layers F.Cu B.Cu) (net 13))
 (segment (start 151.13 91.694) (end 151.13 85.09) (width 0.25) (layer B.Cu) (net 13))
 (segment (start 151.638 92.202) (end 151.13 91.694) (width 0.25) (layer B.Cu) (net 13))
 (via (at 151.638 92.202) (size 0.6) (drill 0.4) (layers F.Cu B.Cu) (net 13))
 (segment (start 153.162 92.202) (end 151.638 92.202) (width 0.25) (layer F.Cu) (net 13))
 (via (at 153.162 92.202) (size 0.6) (drill 0.4) (layers F.Cu B.Cu) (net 13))
 (segment (start 154.686 92.202) (end 153.162 92.202) (width 0.25) (layer B.Cu) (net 13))
 (via (at 154.686 92.202) (size 0.6) (drill 0.4) (layers F.Cu B.Cu) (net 13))
 (segment (start 158.496 92.202) (end 154.686 92.202) (width 0.25) (layer F.Cu) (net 13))
 (segment (start 158.75 91.948) (end 158.496 92.202) (width 0.25) (layer F.Cu) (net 13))
 (via (at 158.75 91.948) (size 0.6) (drill 0.4) (layers F.Cu B.Cu) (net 13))
 (segment (start 158.75 90.932) (end 158.75 91.948) (width 0.25) (layer B.Cu) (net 13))
 (segment (start 159.258 90.424) (end 158.75 90.932) (width 0.25) (layer B.Cu) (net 13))
 (via (at 159.258 90.424) (size 0.6) (drill 0.4) (layers F.Cu B.Cu) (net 13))
 (segment (start 159.496 90.186) (end 159.258 90.424) (width 0.25) (layer F.Cu) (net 13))
 (segment (start 150.876 78.96098) (end 151.35098 78.486) (width 0.25) (layer F.Cu) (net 13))
 (segment (start 185.42 90.932) (end 186.182 90.932) (width 0.25) (layer B.Cu) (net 14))
 (segment (start 186.182 90.932) (end 187.198 89.662) (width 0.25) (layer B.Cu) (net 14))
 (segment (start 187.212941 78.426235) (end 186.436 78.232) (width 0.25) (layer F.Cu) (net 14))
 (segment (start 187.198 84.582) (end 187.212941 78.426235) (width 0.25) (layer F.Cu) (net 14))
 (via (at 187.198 84.582) (size 0.6) (drill 0.4) (layers F.Cu B.Cu) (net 14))
 (segment (start 187.198 89.662) (end 187.198 84.582) (width 0.25) (layer B.Cu) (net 14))
 (segment (start 186.436 78.232) (end 185.42 78.232) (width 0.25) (layer F.Cu) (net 14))
 (segment (start 177.546 97.79) (end 178.308 97.79) (width 0.25) (layer F.Cu) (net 14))
 (segment (start 178.308 97.79) (end 181.864 94.234) (width 0.25) (layer F.Cu) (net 14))
 (via (at 181.864 94.234) (size 0.6) (drill 0.4) (layers F.Cu B.Cu) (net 14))
 (segment (start 181.864 94.234) (end 185.166 90.932) (width 0.25) (layer B.Cu) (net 14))
 (segment (start 185.166 90.932) (end 185.42 90.932) (width 0.25) (layer B.Cu) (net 14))
 (segment (start 157.496 85.157) (end 157.496 84.852) (width 0.25) (layer F.Cu) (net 20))
 (segment (start 157.496 84.852) (end 155.956 83.312) (width 0.25) (layer F.Cu) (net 20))
 (segment (start 155.956 83.312) (end 154.686 83.312) (width 0.25) (layer F.Cu) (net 20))
 (segment (start 154.686 83.312) (end 153.416 82.042) (width 0.25) (layer F.Cu) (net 20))
 (segment (start 153.416 82.042) (end 153.416 80.264) (width 0.25) (layer F.Cu) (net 20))
 (via (at 153.416 80.264) (size 0.6) (drill 0.4) (layers F.Cu B.Cu) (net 20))
 (segment (start 153.416 80.264) (end 153.67 80.01) (width 0.25) (layer B.Cu) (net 20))
 (segment (start 153.67 80.01) (end 169.164 80.01) (width 0.25) (layer B.Cu) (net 20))
 (segment (start 169.164 80.01) (end 170.688 81.534) (width 0.25) (layer B.Cu) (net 20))
 (segment (start 170.688 81.534) (end 184.658 81.534) (width 0.25) (layer B.Cu) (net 20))
 (segment (start 184.658 81.534) (end 185.42 80.772) (width 0.25) (layer B.Cu) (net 20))
 (segment (start 156.531 87.622) (end 155.456 87.622) (width 0.25) (layer F.Cu) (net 21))
 (segment (start 183.134 83.312) (end 185.42 83.312) (width 0.25) (layer B.Cu) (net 21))
 (segment (start 182.118 82.296) (end 183.134 83.312) (width 0.25) (layer B.Cu) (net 21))
 (segment (start 154.686 82.296) (end 182.118 82.296) (width 0.25) (layer B.Cu) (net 21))
 (segment (start 154.686 87.376) (end 154.686 82.296) (width 0.25) (layer B.Cu) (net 21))
 (segment (start 155.194 87.884) (end 154.686 87.376) (width 0.25) (layer B.Cu) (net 21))
 (via (at 155.194 87.884) (size 0.6) (drill 0.4) (layers F.Cu B.Cu) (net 21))
 (segment (start 155.456 87.622) (end 155.194 87.884) (width 0.25) (layer F.Cu) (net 21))
 (segment (start 182.36 88.392) (end 183.388 88.392) (width 0.25) (layer F.Cu) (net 22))
 (segment (start 183.388 88.392) (end 185.42 88.392) (width 0.25) (layer B.Cu) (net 22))
 (via (at 183.388 88.392) (size 0.6) (drill 0.4) (layers F.Cu B.Cu) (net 22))
 (segment (start 141.36116 93.35008) (end 146.86026 93.35008) (width 0.25) (layer F.Cu) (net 24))
 (segment (start 141.36116 84.44992) (end 141.36116 93.35008) (width 0.25) (layer F.Cu) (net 24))
 (segment (start 146.86026 84.44992) (end 141.36116 84.44992) (width 0.25) (layer F.Cu) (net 24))
 (segment (start 160.461 87.622) (end 164.346 87.622) (width 0.25) (layer F.Cu) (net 25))
 (segment (start 165.862 86.106) (end 168.414 86.106) (width 0.25) (layer F.Cu) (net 25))
 (segment (start 164.346 87.622) (end 165.862 86.106) (width 0.25) (layer F.Cu) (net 25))
 (segment (start 160.461 88.122) (end 169.434 88.122) (width 0.25) (layer F.Cu) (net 26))
 (segment (start 172.224 87.364) (end 172.224 86.106) (width 0.25) (layer F.Cu) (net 26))
 (segment (start 171.958 87.63) (end 172.224 87.364) (width 0.25) (layer F.Cu) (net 26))
 (via (at 171.958 87.63) (size 0.6) (drill 0.4) (layers F.Cu B.Cu) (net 26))
 (segment (start 169.926 87.63) (end 171.958 87.63) (width 0.25) (layer B.Cu) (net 26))
 (via (at 169.926 87.63) (size 0.6) (drill 0.4) (layers F.Cu B.Cu) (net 26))
 (segment (start 169.434 88.122) (end 169.926 87.63) (width 0.25) (layer F.Cu) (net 26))
 (segment (start 157.996 85.157) (end 157.996 84.082) (width 0.25) (layer F.Cu) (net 27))
 (segment (start 161.81 79.756) (end 162.826 80.772) (width 0.25) (layer F.Cu) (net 27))
 (segment (start 155.194 79.756) (end 161.81 79.756) (width 0.25) (layer F.Cu) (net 27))
 (segment (start 154.432 80.518) (end 155.194 79.756) (width 0.25) (layer F.Cu) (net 27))
 (segment (start 154.432 82.296) (end 154.432 80.518) (width 0.25) (layer F.Cu) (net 27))
 (segment (start 154.686 82.55) (end 154.432 82.296) (width 0.25) (layer F.Cu) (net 27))
 (segment (start 157.226 82.55) (end 154.686 82.55) (width 0.25) (layer F.Cu) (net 27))
 (segment (start 157.226 83.312) (end 157.226 82.55) (width 0.25) (layer F.Cu) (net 27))
 (segment (start 157.996 84.082) (end 157.226 83.312) (width 0.25) (layer F.Cu) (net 27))
 (segment (start 180.86 88.392) (end 180.86 83.324) (width 0.25) (layer F.Cu) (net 28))
 (segment (start 158.496 83.312) (end 158.496 85.157) (width 0.25) (layer F.Cu) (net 28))
 (segment (start 158.242 83.058) (end 158.496 83.312) (width 0.25) (layer F.Cu) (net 28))
 (via (at 158.242 83.058) (size 0.6) (drill 0.4) (layers F.Cu B.Cu) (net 28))
 (segment (start 180.594 83.058) (end 158.242 83.058) (width 0.25) (layer B.Cu) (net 28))
 (segment (start 180.848 83.312) (end 180.594 83.058) (width 0.25) (layer B.Cu) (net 28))
 (via (at 180.848 83.312) (size 0.6) (drill 0.4) (layers F.Cu B.Cu) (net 28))
 (segment (start 180.86 83.324) (end 180.848 83.312) (width 0.25) (layer F.Cu) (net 28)))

